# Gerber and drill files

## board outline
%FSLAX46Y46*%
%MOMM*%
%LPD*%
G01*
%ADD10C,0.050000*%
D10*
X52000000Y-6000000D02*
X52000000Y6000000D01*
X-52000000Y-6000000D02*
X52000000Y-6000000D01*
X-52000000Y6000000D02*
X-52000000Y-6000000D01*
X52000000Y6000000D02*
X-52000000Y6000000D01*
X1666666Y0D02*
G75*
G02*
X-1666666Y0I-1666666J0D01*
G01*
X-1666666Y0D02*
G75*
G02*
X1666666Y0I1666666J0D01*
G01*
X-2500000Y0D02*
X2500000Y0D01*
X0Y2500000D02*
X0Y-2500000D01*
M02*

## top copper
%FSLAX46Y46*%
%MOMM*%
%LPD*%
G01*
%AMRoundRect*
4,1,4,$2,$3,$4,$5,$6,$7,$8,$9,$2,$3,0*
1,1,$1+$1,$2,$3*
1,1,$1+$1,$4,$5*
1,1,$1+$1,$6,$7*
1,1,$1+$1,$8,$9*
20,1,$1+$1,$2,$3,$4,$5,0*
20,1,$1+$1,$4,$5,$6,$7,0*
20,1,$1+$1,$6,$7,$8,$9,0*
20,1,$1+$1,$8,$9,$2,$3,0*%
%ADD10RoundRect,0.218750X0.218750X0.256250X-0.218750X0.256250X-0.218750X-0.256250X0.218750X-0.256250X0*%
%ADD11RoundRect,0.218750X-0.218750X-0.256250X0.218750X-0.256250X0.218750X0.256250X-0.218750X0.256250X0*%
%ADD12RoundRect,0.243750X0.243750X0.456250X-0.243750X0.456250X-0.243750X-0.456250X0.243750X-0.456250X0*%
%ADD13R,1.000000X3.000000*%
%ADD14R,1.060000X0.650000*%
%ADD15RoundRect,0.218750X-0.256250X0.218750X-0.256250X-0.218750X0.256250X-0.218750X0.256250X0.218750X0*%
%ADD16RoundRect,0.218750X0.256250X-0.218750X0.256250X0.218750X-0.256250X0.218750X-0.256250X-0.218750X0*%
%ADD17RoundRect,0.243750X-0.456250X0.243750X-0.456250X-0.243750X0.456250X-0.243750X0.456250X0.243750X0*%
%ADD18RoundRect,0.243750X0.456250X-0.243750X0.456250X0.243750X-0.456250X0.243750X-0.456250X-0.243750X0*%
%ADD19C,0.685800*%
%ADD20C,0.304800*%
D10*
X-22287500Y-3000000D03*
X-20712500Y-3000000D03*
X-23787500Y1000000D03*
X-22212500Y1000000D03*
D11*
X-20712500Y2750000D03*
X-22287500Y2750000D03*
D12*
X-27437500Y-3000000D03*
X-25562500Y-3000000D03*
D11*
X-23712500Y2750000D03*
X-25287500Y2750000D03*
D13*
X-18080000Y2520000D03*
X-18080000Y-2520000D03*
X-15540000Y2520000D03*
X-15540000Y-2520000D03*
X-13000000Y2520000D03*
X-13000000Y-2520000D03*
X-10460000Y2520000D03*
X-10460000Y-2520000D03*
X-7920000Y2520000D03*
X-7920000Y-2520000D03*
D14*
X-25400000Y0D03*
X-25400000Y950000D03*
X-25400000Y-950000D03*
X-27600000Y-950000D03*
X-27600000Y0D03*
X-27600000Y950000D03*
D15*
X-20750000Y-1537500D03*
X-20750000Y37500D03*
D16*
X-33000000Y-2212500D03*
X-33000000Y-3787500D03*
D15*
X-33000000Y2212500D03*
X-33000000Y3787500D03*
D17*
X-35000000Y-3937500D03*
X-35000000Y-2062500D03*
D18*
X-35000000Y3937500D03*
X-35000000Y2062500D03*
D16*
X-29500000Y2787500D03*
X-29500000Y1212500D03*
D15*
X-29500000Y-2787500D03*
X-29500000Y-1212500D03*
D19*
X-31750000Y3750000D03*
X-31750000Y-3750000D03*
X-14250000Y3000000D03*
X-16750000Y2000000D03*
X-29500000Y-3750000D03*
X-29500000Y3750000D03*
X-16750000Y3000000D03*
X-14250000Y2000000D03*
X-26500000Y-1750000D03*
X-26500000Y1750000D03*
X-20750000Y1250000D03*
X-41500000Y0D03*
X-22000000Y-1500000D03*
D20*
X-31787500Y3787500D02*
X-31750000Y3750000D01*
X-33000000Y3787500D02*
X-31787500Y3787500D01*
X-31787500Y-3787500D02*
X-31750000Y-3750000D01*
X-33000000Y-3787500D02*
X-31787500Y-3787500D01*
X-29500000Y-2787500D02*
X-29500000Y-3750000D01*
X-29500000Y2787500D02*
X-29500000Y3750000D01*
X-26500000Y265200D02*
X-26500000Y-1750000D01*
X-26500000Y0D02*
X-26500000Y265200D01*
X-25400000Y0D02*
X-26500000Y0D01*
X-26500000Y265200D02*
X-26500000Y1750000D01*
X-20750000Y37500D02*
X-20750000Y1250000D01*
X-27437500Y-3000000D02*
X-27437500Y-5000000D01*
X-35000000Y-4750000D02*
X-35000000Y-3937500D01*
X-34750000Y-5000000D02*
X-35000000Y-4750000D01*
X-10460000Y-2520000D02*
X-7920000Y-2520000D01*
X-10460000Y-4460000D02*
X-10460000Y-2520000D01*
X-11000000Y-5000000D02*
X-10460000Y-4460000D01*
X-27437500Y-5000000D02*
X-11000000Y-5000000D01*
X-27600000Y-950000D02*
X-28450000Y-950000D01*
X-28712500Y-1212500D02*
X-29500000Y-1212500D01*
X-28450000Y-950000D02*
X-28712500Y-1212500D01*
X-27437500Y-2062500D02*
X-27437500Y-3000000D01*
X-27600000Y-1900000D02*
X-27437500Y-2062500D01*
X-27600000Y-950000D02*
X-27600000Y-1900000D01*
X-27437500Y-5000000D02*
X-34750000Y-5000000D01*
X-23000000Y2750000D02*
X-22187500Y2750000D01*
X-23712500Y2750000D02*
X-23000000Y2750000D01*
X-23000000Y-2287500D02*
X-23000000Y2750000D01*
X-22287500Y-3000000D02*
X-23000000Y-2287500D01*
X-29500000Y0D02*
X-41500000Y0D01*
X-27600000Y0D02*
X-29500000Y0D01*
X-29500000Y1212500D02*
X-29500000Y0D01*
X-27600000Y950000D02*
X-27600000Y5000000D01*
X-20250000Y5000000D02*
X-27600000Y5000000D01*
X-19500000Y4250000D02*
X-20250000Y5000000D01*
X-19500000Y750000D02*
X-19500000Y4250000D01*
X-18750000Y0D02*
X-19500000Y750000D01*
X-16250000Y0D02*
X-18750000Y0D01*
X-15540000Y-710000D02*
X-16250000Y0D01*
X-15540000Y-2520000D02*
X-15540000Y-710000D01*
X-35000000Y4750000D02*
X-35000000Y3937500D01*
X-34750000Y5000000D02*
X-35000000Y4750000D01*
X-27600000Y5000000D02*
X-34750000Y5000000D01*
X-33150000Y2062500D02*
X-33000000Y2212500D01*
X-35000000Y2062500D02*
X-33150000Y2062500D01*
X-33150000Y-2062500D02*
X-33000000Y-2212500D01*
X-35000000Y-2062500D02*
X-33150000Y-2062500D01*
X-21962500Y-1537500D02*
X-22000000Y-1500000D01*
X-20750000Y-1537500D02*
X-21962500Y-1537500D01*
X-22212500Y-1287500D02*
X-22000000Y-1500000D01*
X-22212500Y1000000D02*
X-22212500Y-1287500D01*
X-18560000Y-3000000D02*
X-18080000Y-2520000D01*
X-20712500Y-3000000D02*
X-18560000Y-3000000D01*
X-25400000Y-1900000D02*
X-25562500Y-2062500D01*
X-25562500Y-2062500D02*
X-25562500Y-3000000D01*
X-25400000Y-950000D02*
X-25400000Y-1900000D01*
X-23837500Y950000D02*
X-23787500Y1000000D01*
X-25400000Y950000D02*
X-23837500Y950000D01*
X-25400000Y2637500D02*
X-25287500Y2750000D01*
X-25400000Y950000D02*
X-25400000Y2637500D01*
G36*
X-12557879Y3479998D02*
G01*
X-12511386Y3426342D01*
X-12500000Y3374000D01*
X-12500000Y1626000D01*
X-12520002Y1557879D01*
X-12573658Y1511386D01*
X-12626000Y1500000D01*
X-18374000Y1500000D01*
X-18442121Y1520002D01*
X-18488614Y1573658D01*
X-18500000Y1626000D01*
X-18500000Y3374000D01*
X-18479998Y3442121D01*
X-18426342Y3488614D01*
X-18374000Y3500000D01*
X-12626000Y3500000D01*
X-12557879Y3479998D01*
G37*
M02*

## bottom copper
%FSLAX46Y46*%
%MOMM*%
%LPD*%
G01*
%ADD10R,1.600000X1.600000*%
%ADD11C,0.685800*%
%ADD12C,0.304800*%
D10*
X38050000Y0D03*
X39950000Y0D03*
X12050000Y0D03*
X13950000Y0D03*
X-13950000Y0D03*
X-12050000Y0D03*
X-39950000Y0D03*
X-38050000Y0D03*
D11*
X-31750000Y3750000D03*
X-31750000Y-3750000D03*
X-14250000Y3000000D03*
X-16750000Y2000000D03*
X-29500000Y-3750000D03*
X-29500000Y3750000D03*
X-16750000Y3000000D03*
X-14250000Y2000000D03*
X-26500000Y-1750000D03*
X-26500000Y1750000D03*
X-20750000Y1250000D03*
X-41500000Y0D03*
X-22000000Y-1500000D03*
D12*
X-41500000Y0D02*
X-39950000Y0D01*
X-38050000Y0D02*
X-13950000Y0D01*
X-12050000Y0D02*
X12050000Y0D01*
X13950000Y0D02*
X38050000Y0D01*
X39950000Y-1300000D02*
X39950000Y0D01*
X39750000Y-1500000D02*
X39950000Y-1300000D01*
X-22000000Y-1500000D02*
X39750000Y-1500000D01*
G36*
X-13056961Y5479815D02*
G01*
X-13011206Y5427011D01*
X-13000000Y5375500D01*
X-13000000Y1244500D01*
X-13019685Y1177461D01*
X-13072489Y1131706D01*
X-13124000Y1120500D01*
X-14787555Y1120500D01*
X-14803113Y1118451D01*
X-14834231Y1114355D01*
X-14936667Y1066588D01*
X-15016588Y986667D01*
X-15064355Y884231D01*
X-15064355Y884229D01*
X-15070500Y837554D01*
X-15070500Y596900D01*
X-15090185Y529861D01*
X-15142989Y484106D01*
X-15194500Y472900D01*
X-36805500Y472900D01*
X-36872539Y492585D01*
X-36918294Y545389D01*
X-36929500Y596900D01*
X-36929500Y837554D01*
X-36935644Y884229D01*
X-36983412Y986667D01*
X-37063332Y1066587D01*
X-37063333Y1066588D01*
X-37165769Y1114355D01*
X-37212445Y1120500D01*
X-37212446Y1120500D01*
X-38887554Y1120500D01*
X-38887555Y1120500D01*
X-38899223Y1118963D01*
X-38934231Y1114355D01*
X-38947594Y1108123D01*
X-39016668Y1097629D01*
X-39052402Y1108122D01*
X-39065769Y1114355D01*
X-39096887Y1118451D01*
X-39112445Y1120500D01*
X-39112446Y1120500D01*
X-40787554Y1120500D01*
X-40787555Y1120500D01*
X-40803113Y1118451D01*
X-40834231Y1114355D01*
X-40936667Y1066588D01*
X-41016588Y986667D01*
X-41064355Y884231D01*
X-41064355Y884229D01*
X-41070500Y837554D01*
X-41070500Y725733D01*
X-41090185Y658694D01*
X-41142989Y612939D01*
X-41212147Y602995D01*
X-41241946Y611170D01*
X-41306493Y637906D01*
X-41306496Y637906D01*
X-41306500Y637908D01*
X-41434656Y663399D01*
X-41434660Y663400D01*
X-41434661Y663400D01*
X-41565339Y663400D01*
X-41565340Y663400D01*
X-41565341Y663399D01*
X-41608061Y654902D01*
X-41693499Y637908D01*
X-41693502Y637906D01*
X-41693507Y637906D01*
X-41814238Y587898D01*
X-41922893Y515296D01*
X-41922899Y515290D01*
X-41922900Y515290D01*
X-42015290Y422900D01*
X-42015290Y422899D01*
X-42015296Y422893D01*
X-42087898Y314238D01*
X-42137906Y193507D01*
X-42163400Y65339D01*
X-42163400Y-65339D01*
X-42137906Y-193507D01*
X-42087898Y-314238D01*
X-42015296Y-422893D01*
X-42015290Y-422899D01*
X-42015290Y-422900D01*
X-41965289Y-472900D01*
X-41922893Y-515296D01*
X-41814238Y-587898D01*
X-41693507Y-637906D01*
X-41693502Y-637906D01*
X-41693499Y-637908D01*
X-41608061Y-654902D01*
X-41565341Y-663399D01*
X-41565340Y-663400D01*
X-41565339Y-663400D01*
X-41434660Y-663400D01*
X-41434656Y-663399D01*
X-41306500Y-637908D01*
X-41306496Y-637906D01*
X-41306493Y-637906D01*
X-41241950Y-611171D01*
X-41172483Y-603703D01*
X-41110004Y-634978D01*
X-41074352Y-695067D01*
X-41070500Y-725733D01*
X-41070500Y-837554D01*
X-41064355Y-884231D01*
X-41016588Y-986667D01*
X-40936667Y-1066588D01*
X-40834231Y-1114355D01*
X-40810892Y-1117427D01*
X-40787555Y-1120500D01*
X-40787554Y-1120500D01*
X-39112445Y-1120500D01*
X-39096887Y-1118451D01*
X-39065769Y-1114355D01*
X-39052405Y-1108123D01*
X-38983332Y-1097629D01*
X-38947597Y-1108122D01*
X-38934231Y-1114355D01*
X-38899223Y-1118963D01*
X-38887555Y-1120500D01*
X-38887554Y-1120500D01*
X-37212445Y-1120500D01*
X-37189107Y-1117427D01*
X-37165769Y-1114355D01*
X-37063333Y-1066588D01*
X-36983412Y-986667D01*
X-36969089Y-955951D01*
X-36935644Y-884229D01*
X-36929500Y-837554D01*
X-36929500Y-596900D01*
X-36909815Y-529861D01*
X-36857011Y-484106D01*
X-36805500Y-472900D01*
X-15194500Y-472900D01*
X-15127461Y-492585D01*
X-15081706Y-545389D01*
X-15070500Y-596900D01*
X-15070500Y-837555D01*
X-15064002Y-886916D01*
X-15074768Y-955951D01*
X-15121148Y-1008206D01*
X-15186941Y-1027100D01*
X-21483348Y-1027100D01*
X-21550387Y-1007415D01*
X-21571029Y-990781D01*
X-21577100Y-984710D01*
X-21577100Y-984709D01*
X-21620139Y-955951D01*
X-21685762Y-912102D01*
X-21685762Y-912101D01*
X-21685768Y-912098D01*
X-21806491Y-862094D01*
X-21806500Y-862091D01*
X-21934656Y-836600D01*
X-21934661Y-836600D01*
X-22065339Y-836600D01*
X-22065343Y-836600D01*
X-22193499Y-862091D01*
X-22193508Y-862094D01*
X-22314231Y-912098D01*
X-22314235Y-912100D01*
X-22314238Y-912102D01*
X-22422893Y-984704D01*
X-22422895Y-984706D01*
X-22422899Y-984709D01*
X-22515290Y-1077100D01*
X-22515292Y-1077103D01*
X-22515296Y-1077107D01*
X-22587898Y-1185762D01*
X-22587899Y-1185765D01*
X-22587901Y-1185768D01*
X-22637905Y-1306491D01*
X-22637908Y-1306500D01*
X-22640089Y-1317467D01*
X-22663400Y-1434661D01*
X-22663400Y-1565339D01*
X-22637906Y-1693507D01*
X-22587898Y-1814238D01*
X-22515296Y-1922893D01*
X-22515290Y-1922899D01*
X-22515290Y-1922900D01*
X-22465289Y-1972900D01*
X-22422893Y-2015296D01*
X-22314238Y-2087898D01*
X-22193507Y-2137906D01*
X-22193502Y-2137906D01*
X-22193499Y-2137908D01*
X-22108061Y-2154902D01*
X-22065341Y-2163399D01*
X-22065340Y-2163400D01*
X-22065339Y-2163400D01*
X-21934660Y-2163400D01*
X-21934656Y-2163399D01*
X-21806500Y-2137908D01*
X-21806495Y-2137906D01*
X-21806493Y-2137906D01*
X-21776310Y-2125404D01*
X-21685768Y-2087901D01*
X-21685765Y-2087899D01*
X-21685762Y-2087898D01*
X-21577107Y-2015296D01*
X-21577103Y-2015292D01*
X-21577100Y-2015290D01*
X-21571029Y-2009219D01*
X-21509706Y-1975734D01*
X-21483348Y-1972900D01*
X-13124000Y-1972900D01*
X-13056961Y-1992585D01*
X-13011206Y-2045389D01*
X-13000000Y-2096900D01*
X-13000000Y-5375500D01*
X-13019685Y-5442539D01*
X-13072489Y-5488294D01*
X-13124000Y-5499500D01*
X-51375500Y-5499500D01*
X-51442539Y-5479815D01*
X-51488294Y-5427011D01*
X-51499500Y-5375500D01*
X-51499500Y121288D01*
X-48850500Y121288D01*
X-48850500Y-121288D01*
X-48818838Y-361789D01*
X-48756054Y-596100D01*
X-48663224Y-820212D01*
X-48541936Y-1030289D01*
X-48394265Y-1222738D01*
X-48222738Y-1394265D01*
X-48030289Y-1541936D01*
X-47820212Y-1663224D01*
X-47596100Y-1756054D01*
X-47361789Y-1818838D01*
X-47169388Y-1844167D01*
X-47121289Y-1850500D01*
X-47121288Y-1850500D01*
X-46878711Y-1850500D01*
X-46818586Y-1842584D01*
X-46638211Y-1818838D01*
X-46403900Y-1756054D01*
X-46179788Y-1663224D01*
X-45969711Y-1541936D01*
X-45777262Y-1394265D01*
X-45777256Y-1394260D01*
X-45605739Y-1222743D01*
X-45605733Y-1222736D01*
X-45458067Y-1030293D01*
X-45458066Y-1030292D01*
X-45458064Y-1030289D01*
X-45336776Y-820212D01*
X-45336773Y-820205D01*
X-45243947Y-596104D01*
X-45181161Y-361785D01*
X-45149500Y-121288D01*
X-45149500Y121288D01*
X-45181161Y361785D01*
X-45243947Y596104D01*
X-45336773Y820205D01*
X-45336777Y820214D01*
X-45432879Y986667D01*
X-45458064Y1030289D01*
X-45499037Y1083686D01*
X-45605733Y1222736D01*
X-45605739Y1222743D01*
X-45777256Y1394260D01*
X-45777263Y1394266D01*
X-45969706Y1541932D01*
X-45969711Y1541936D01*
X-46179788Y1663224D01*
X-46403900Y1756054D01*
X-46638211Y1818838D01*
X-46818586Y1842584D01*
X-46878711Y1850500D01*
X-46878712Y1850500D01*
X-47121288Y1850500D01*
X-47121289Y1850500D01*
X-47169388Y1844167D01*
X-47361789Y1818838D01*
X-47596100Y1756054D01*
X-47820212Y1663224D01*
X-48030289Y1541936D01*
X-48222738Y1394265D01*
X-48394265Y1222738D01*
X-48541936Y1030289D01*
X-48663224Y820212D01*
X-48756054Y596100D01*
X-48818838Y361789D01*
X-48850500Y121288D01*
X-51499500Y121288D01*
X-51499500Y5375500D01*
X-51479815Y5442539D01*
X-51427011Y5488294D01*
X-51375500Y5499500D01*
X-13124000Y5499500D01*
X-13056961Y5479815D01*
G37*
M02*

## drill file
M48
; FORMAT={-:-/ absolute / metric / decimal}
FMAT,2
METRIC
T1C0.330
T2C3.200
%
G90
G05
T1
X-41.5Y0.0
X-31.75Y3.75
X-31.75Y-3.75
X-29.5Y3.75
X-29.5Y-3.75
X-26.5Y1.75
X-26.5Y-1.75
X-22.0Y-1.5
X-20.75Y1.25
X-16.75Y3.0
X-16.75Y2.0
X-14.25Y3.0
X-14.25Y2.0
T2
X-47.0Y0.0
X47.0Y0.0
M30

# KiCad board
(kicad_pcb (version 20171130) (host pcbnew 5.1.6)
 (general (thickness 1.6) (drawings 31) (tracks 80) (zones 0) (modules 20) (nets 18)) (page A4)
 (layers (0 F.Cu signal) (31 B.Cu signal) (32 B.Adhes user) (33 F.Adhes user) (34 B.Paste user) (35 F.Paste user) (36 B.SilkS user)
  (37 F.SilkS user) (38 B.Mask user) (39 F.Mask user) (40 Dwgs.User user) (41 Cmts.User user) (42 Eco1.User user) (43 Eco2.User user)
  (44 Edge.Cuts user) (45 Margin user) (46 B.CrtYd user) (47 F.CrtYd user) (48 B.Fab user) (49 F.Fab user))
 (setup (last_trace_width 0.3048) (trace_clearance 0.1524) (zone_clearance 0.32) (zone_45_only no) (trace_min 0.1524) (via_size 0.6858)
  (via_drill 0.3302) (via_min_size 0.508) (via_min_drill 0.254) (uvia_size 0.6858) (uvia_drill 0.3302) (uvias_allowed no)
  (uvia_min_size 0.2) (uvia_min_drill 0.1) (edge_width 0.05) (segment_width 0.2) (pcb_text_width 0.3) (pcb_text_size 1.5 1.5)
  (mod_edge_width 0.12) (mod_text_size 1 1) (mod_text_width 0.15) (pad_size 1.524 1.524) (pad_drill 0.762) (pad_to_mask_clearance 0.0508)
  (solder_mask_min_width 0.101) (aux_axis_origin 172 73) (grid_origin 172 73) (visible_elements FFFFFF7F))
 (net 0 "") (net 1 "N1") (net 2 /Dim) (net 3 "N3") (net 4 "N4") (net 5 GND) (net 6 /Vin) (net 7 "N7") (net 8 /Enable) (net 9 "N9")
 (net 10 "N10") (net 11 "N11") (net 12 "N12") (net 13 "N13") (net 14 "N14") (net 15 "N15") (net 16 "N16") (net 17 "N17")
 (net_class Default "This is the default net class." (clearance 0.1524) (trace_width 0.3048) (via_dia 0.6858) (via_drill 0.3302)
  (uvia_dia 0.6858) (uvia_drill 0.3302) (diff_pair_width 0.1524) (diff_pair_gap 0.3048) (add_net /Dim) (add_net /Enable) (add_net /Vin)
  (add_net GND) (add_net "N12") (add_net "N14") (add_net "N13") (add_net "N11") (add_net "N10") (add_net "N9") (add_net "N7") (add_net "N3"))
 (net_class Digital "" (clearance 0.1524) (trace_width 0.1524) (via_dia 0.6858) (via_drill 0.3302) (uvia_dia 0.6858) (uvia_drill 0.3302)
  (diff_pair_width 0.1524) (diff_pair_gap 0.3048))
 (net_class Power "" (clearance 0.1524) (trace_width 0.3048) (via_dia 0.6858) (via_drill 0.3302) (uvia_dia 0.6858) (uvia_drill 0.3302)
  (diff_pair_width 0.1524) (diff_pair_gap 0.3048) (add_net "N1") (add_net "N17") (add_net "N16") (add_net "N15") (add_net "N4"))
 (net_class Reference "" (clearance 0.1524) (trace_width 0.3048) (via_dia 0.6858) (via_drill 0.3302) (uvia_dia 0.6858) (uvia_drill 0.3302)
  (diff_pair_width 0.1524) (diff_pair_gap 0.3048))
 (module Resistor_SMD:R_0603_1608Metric (layer F.Cu) (at -21.5 3 180)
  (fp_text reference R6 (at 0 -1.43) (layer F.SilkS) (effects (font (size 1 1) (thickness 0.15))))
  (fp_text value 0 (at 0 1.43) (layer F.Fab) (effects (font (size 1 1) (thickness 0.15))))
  (pad 2 smd roundrect (at 0.7875 0 180) (size 0.875 0.95) (layers F.Cu F.Paste F.Mask) (roundrect_rratio 0.25) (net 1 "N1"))
  (pad 1 smd roundrect (at -0.7875 0 180) (size 0.875 0.95) (layers F.Cu F.Paste F.Mask) (roundrect_rratio 0.25) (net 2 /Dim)))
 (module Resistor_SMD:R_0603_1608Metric (layer F.Cu) (at -23 -1 180)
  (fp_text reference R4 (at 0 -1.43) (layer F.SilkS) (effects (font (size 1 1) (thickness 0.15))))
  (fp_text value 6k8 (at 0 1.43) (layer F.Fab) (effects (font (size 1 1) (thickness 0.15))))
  (pad 2 smd roundrect (at 0.7875 0 180) (size 0.875 0.95) (layers F.Cu F.Paste F.Mask) (roundrect_rratio 0.25) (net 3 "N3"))
  (pad 1 smd roundrect (at -0.7875 0 180) (size 0.875 0.95) (layers F.Cu F.Paste F.Mask) (roundrect_rratio 0.25) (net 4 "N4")))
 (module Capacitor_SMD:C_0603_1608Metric (layer F.Cu) (at -21.5 -2.75)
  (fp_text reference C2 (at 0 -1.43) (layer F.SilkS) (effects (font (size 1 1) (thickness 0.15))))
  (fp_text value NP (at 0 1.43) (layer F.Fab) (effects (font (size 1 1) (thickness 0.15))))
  (pad 2 smd roundrect (at 0.7875 0) (size 0.875 0.95) (layers F.Cu F.Paste F.Mask) (roundrect_rratio 0.25) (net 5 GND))
  (pad 1 smd roundrect (at -0.7875 0) (size 0.875 0.95) (layers F.Cu F.Paste F.Mask) (roundrect_rratio 0.25) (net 1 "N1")))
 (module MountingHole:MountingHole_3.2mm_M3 (layer F.Cu) (at -47 0)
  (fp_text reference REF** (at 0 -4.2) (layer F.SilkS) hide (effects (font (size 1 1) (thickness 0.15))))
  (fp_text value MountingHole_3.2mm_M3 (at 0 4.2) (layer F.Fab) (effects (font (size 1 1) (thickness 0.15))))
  (pad 1 np_thru_hole circle (at 0 0) (size 3.2 3.2) (drill 3.2) (layers *.Cu *.Mask)))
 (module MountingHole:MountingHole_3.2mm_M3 (layer F.Cu) (at 47 0)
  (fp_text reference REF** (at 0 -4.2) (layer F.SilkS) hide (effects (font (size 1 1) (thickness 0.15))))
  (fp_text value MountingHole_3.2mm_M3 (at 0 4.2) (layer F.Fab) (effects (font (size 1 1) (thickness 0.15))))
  (pad 1 np_thru_hole circle (at 0 0) (size 3.2 3.2) (drill 3.2) (layers *.Cu *.Mask)))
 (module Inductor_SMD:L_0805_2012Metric (layer F.Cu) (at -26.5 3 180)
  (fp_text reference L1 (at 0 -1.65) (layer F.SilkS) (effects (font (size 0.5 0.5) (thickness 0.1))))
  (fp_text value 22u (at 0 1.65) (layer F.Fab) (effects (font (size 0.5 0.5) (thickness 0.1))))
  (pad 2 smd roundrect (at 0.9375 0 180) (size 0.975 1.4) (layers F.Cu F.Paste F.Mask) (roundrect_rratio 0.25) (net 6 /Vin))
  (pad 1 smd roundrect (at -0.9375 0 180) (size 0.975 1.4) (layers F.Cu F.Paste F.Mask) (roundrect_rratio 0.25) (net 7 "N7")))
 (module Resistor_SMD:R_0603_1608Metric (layer F.Cu) (at -24.5 -2.75)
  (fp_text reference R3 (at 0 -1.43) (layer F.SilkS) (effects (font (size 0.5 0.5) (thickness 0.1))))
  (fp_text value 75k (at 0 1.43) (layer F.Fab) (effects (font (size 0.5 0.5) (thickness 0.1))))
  (pad 2 smd roundrect (at 0.7875 0) (size 0.875 0.95) (layers F.Cu F.Paste F.Mask) (roundrect_rratio 0.25) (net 1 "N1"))
  (pad 1 smd roundrect (at -0.7875 0) (size 0.875 0.95) (layers F.Cu F.Paste F.Mask) (roundrect_rratio 0.25) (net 3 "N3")))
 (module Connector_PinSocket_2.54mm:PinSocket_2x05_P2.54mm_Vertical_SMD (layer F.Cu) (at -13 0 270)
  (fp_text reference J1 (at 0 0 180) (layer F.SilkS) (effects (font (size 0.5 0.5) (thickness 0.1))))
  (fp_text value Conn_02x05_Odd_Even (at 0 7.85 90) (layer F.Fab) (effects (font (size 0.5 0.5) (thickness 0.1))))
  (pad 10 smd rect (at -2.52 5.08 270) (size 3 1) (layers F.Cu F.Paste F.Mask) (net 5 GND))
  (pad 9 smd rect (at 2.52 5.08 270) (size 3 1) (layers F.Cu F.Paste F.Mask) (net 2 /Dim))
  (pad 8 smd rect (at -2.52 2.54 270) (size 3 1) (layers F.Cu F.Paste F.Mask) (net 5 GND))
  (pad 7 smd rect (at 2.52 2.54 270) (size 3 1) (layers F.Cu F.Paste F.Mask) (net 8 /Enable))
  (pad 6 smd rect (at -2.52 0 270) (size 3 1) (layers F.Cu F.Paste F.Mask) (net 5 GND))
  (pad 5 smd rect (at 2.52 0 270) (size 3 1) (layers F.Cu F.Paste F.Mask) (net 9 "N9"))
  (pad 4 smd rect (at -2.52 -2.54 270) (size 3 1) (layers F.Cu F.Paste F.Mask) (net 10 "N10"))
  (pad 3 smd rect (at 2.52 -2.54 270) (size 3 1) (layers F.Cu F.Paste F.Mask) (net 6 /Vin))
  (pad 2 smd rect (at -2.52 -5.08 270) (size 3 1) (layers F.Cu F.Paste F.Mask) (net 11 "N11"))
  (pad 1 smd rect (at 2.52 -5.08 270) (size 3 1) (layers F.Cu F.Paste F.Mask) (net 6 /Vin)))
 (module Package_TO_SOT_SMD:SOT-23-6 (layer F.Cu) (at -26.5 0)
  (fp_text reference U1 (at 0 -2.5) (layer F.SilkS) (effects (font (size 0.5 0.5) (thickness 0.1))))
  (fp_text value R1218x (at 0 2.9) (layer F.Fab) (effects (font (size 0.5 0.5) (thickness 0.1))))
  (pad 5 smd rect (at 1.1 0) (size 1.06 0.65) (layers F.Cu F.Paste F.Mask) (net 5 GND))
  (pad 6 smd rect (at 1.1 -0.95) (size 1.06 0.65) (layers F.Cu F.Paste F.Mask) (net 3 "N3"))
  (pad 4 smd rect (at 1.1 0.95) (size 1.06 0.65) (layers F.Cu F.Paste F.Mask) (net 7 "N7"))
  (pad 3 smd rect (at -1.1 0.95) (size 1.06 0.65) (layers F.Cu F.Paste F.Mask) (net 6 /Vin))
  (pad 2 smd rect (at -1.1 0) (size 1.06 0.65) (layers F.Cu F.Paste F.Mask) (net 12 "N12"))
  (pad 1 smd rect (at -1.1 -0.95) (size 1.06 0.65) (layers F.Cu F.Paste F.Mask) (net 8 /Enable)))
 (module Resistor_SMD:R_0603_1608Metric (layer F.Cu) (at -20.75 0.75 270)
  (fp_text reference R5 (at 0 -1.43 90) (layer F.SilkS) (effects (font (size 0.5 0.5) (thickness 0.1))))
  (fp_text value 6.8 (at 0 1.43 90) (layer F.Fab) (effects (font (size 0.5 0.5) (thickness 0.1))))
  (pad 2 smd roundrect (at 0.7875 0 270) (size 0.875 0.95) (layers F.Cu F.Paste F.Mask) (roundrect_rratio 0.25) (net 4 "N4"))
  (pad 1 smd roundrect (at -0.7875 0 270) (size 0.875 0.95) (layers F.Cu F.Paste F.Mask) (roundrect_rratio 0.25) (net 5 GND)))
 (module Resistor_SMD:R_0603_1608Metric (layer F.Cu) (at -33 3 90)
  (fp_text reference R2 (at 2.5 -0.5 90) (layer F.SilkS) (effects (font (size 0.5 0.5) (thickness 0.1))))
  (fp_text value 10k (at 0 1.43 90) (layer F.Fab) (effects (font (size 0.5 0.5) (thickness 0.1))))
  (pad 2 smd roundrect (at 0.7875 0 90) (size 0.875 0.95) (layers F.Cu F.Paste F.Mask) (roundrect_rratio 0.25) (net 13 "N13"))
  (pad 1 smd roundrect (at -0.7875 0 90) (size 0.875 0.95) (layers F.Cu F.Paste F.Mask) (roundrect_rratio 0.25) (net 5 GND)))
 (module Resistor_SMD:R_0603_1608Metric (layer F.Cu) (at -33 -3 270)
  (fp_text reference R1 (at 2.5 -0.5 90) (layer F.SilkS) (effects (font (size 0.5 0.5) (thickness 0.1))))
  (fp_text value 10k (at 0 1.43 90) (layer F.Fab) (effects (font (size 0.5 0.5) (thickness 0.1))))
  (pad 2 smd roundrect (at 0.7875 0 270) (size 0.875 0.95) (layers F.Cu F.Paste F.Mask) (roundrect_rratio 0.25) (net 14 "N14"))
  (pad 1 smd roundrect (at -0.7875 0 270) (size 0.875 0.95) (layers F.Cu F.Paste F.Mask) (roundrect_rratio 0.25) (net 5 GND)))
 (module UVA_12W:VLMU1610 (layer B.Cu) (at 39 0 180)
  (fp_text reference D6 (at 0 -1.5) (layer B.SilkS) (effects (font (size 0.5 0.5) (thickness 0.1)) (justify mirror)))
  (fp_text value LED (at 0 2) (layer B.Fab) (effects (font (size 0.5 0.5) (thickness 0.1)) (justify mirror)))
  (pad 2 smd rect (at 0.95 0 180) (size 1.6 1.6) (layers B.Cu B.Paste B.Mask) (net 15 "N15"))
  (pad 1 smd rect (at -0.95 0 180) (size 1.6 1.6) (layers B.Cu B.Paste B.Mask) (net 4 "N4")))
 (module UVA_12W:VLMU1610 (layer B.Cu) (at 13 0 180)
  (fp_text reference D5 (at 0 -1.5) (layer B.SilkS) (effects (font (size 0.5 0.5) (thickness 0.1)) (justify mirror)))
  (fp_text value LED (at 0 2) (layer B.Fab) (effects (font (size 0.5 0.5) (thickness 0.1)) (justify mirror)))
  (pad 2 smd rect (at 0.95 0 180) (size 1.6 1.6) (layers B.Cu B.Paste B.Mask) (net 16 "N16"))
  (pad 1 smd rect (at -0.95 0 180) (size 1.6 1.6) (layers B.Cu B.Paste B.Mask) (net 15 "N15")))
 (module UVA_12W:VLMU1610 (layer B.Cu) (at -13 0 180)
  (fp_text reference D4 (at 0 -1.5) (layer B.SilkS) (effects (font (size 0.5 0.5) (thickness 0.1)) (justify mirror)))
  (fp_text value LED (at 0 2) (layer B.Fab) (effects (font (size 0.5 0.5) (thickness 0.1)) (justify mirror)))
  (pad 2 smd rect (at 0.95 0 180) (size 1.6 1.6) (layers B.Cu B.Paste B.Mask) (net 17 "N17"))
  (pad 1 smd rect (at -0.95 0 180) (size 1.6 1.6) (layers B.Cu B.Paste B.Mask) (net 16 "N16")))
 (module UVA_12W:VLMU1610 (layer B.Cu) (at -39 0 180)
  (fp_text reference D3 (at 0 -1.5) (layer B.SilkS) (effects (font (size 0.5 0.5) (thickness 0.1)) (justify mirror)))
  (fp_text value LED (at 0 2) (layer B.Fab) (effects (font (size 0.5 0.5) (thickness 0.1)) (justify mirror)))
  (pad 2 smd rect (at 0.95 0 180) (size 1.6 1.6) (layers B.Cu B.Paste B.Mask) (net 12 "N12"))
  (pad 1 smd rect (at -0.95 0 180) (size 1.6 1.6) (layers B.Cu B.Paste B.Mask) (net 17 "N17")))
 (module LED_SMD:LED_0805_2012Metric (layer F.Cu) (at -35 3 270)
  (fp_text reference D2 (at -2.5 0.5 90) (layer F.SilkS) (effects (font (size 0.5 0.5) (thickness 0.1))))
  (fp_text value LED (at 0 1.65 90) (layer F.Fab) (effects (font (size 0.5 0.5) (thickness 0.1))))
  (pad 2 smd roundrect (at 0.9375 0 270) (size 0.975 1.4) (layers F.Cu F.Paste F.Mask) (roundrect_rratio 0.25) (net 6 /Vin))
  (pad 1 smd roundrect (at -0.9375 0 270) (size 0.975 1.4) (layers F.Cu F.Paste F.Mask) (roundrect_rratio 0.25) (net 13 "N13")))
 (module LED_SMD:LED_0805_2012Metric (layer F.Cu) (at -35 -3 90)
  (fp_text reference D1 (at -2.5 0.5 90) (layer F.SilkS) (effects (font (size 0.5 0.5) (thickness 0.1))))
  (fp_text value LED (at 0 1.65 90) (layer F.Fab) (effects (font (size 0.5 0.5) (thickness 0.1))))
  (pad 2 smd roundrect (at 0.9375 0 90) (size 0.975 1.4) (layers F.Cu F.Paste F.Mask) (roundrect_rratio 0.25) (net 8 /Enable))
  (pad 1 smd roundrect (at -0.9375 0 90) (size 0.975 1.4) (layers F.Cu F.Paste F.Mask) (roundrect_rratio 0.25) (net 14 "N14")))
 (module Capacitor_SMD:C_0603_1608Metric (layer F.Cu) (at -29.5 -2 90)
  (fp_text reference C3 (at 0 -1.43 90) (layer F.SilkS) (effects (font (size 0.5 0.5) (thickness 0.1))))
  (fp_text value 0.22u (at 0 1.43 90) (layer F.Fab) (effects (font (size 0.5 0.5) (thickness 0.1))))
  (pad 2 smd roundrect (at 0.7875 0 90) (size 0.875 0.95) (layers F.Cu F.Paste F.Mask) (roundrect_rratio 0.25) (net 5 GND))
  (pad 1 smd roundrect (at -0.7875 0 90) (size 0.875 0.95) (layers F.Cu F.Paste F.Mask) (roundrect_rratio 0.25) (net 12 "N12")))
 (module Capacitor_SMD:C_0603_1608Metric (layer F.Cu) (at -29.5 2 270)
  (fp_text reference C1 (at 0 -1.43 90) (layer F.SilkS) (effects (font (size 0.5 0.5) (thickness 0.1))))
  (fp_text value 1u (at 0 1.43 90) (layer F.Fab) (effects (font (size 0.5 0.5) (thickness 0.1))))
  (pad 2 smd roundrect (at 0.7875 0 270) (size 0.875 0.95) (layers F.Cu F.Paste F.Mask) (roundrect_rratio 0.25) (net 5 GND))
  (pad 1 smd roundrect (at -0.7875 0 270) (size 0.875 0.95) (layers F.Cu F.Paste F.Mask) (roundrect_rratio 0.25) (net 6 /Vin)))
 (gr_line (start 52 6) (end 52 -6) (layer Edge.Cuts) (width 0.05))
 (gr_line (start -52 6) (end 52 6) (layer Edge.Cuts) (width 0.05))
 (gr_line (start -52 -6) (end -52 6) (layer Edge.Cuts) (width 0.05))
 (gr_line (start 52 -6) (end -52 -6) (layer Edge.Cuts) (width 0.05))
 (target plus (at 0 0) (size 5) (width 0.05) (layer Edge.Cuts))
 (via (at -31.75 -3.75) (size 0.6858) (drill 0.3302) (layers F.Cu B.Cu) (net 5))
 (segment (start -31.7875 -3.7875) (end -31.75 -3.75) (width 0.3048) (layer F.Cu) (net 5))
 (segment (start -33 -3.7875) (end -31.7875 -3.7875) (width 0.3048) (layer F.Cu) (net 5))
 (segment (start -31.7875 3.7875) (end -31.75 3.75) (width 0.3048) (layer F.Cu) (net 5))
 (via (at -31.75 3.75) (size 0.6858) (drill 0.3302) (layers F.Cu B.Cu) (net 5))
 (segment (start -33 3.7875) (end -31.7875 3.7875) (width 0.3048) (layer F.Cu) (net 5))
 (via (at -14.25 -3) (size 0.6858) (drill 0.3302) (layers F.Cu B.Cu) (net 5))
 (via (at -16.75 -2) (size 0.6858) (drill 0.3302) (layers F.Cu B.Cu) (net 5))
 (via (at -29.5 3.75) (size 0.6858) (drill 0.3302) (layers F.Cu B.Cu) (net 5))
 (segment (start -29.5 2.7875) (end -29.5 3.75) (width 0.3048) (layer F.Cu) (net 5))
 (via (at -29.5 -3.75) (size 0.6858) (drill 0.3302) (layers F.Cu B.Cu) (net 5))
 (segment (start -29.5 -2.7875) (end -29.5 -3.75) (width 0.3048) (layer F.Cu) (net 5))
 (via (at -16.75 -3) (size 0.6858) (drill 0.3302) (layers F.Cu B.Cu) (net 5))
 (via (at -14.25 -2) (size 0.6858) (drill 0.3302) (layers F.Cu B.Cu) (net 5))
 (via (at -26.5 1.75) (size 0.6858) (drill 0.3302) (layers F.Cu B.Cu) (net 5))
 (segment (start -26.5 -0.2652) (end -26.5 1.75) (width 0.3048) (layer F.Cu) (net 5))
 (segment (start -26.5 0) (end -26.5 -0.2652) (width 0.3048) (layer F.Cu) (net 5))
 (segment (start -25.4 0) (end -26.5 0) (width 0.3048) (layer F.Cu) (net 5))
 (segment (start -26.5 -0.2652) (end -26.5 -1.75) (width 0.3048) (layer F.Cu) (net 5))
 (via (at -26.5 -1.75) (size 0.6858) (drill 0.3302) (layers F.Cu B.Cu) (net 5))
 (via (at -20.75 -1.25) (size 0.6858) (drill 0.3302) (layers F.Cu B.Cu) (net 5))
 (segment (start -20.75 -0.0375) (end -20.75 -1.25) (width 0.3048) (layer F.Cu) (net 5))
 (segment (start -27.4375 3) (end -27.4375 5) (width 0.3048) (layer F.Cu) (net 6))
 (segment (start -35 4.75) (end -35 3.9375) (width 0.3048) (layer F.Cu) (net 6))
 (segment (start -34.75 5) (end -35 4.75) (width 0.3048) (layer F.Cu) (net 6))
 (segment (start -10.46 2.52) (end -7.92 2.52) (width 0.3048) (layer F.Cu) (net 6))
 (segment (start -10.46 4.46) (end -10.46 2.52) (width 0.3048) (layer F.Cu) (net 6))
 (segment (start -11 5) (end -10.46 4.46) (width 0.3048) (layer F.Cu) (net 6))
 (segment (start -27.4375 5) (end -11 5) (width 0.3048) (layer F.Cu) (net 6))
 (segment (start -27.6 0.95) (end -28.45 0.95) (width 0.3048) (layer F.Cu) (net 6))
 (segment (start -28.7125 1.2125) (end -29.5 1.2125) (width 0.3048) (layer F.Cu) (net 6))
 (segment (start -28.45 0.95) (end -28.7125 1.2125) (width 0.3048) (layer F.Cu) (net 6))
 (segment (start -27.4375 2.0625) (end -27.4375 3) (width 0.3048) (layer F.Cu) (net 6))
 (segment (start -27.6 1.9) (end -27.4375 2.0625) (width 0.3048) (layer F.Cu) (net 6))
 (segment (start -27.6 0.95) (end -27.6 1.9) (width 0.3048) (layer F.Cu) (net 6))
 (segment (start -27.4375 5) (end -34.75 5) (width 0.3048) (layer F.Cu) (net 6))
 (segment (start -23 -2.75) (end -22.1875 -2.75) (width 0.3048) (layer F.Cu) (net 1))
 (segment (start -23.7125 -2.75) (end -23 -2.75) (width 0.3048) (layer F.Cu) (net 1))
 (segment (start -23 2.2875) (end -23 -2.75) (width 0.3048) (layer F.Cu) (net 1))
 (segment (start -22.2875 3) (end -23 2.2875) (width 0.3048) (layer F.Cu) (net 1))
 (via (at -41.5 0) (size 0.6858) (drill 0.3302) (layers F.Cu B.Cu) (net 12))
 (segment (start -41.5 0) (end -39.95 0) (width 0.3048) (layer B.Cu) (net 12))
 (segment (start -29.5 0) (end -41.5 0) (width 0.3048) (layer F.Cu) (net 12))
 (segment (start -27.6 0) (end -29.5 0) (width 0.3048) (layer F.Cu) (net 12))
 (segment (start -29.5 -1.2125) (end -29.5 0) (width 0.3048) (layer F.Cu) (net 12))
 (segment (start -27.6 -0.95) (end -27.6 -5) (width 0.3048) (layer F.Cu) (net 8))
 (segment (start -20.25 -5) (end -27.6 -5) (width 0.3048) (layer F.Cu) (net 8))
 (segment (start -19.5 -4.25) (end -20.25 -5) (width 0.3048) (layer F.Cu) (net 8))
 (segment (start -19.5 -0.75) (end -19.5 -4.25) (width 0.3048) (layer F.Cu) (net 8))
 (segment (start -18.75 0) (end -19.5 -0.75) (width 0.3048) (layer F.Cu) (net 8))
 (segment (start -16.25 0) (end -18.75 0) (width 0.3048) (layer F.Cu) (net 8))
 (segment (start -15.54 0.71) (end -16.25 0) (width 0.3048) (layer F.Cu) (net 8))
 (segment (start -15.54 2.52) (end -15.54 0.71) (width 0.3048) (layer F.Cu) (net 8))
 (segment (start -35 -4.75) (end -35 -3.9375) (width 0.3048) (layer F.Cu) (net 8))
 (segment (start -34.75 -5) (end -35 -4.75) (width 0.3048) (layer F.Cu) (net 8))
 (segment (start -27.6 -5) (end -34.75 -5) (width 0.3048) (layer F.Cu) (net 8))
 (segment (start -33.15 -2.0625) (end -33 -2.2125) (width 0.3048) (layer F.Cu) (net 14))
 (segment (start -35 -2.0625) (end -33.15 -2.0625) (width 0.3048) (layer F.Cu) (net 14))
 (segment (start -33.15 2.0625) (end -33 2.2125) (width 0.3048) (layer F.Cu) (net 13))
 (segment (start -35 2.0625) (end -33.15 2.0625) (width 0.3048) (layer F.Cu) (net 13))
 (segment (start -38.05 0) (end -13.95 0) (width 0.3048) (layer B.Cu) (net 17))
 (segment (start -12.05 0) (end 12.05 0) (width 0.3048) (layer B.Cu) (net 16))
 (segment (start 13.95 0) (end 38.05 0) (width 0.3048) (layer B.Cu) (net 15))
 (segment (start 39.95 1.3) (end 39.95 0) (width 0.3048) (layer B.Cu) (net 4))
 (segment (start 39.75 1.5) (end 39.95 1.3) (width 0.3048) (layer B.Cu) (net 4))
 (segment (start -22 1.5) (end 39.75 1.5) (width 0.3048) (layer B.Cu) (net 4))
 (via (at -22 1.5) (size 0.6858) (drill 0.3302) (layers F.Cu B.Cu) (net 4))
 (segment (start -21.9625 1.5375) (end -22 1.5) (width 0.3048) (layer F.Cu) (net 4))
 (segment (start -20.75 1.5375) (end -21.9625 1.5375) (width 0.3048) (layer F.Cu) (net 4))
 (segment (start -22.2125 1.2875) (end -22 1.5) (width 0.3048) (layer F.Cu) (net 4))
 (segment (start -22.2125 -1) (end -22.2125 1.2875) (width 0.3048) (layer F.Cu) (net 4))
 (segment (start -18.56 3) (end -18.08 2.52) (width 0.3048) (layer F.Cu) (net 2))
 (segment (start -20.7125 3) (end -18.56 3) (width 0.3048) (layer F.Cu) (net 2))
 (segment (start -25.4 1.9) (end -25.5625 2.0625) (width 0.3048) (layer F.Cu) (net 7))
 (segment (start -25.5625 2.0625) (end -25.5625 3) (width 0.3048) (layer F.Cu) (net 7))
 (segment (start -25.4 0.95) (end -25.4 1.9) (width 0.3048) (layer F.Cu) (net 7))
 (segment (start -23.8375 -0.95) (end -23.7875 -1) (width 0.3048) (layer F.Cu) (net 3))
 (segment (start -25.4 -0.95) (end -23.8375 -0.95) (width 0.3048) (layer F.Cu) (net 3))
 (segment (start -25.4 -2.6375) (end -25.2875 -2.75) (width 0.3048) (layer F.Cu) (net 3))
 (segment (start -25.4 -0.95) (end -25.4 -2.6375) (width 0.3048) (layer F.Cu) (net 3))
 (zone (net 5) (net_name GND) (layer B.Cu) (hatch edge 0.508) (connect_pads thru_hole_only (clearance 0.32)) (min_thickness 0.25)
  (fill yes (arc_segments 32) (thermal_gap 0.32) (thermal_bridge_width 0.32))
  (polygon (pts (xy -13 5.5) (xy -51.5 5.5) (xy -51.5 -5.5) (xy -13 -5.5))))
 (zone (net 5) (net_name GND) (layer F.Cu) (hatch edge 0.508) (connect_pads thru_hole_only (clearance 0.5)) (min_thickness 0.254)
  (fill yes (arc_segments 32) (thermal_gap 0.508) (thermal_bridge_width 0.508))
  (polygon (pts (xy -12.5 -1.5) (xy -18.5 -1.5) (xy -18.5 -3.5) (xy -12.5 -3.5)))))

